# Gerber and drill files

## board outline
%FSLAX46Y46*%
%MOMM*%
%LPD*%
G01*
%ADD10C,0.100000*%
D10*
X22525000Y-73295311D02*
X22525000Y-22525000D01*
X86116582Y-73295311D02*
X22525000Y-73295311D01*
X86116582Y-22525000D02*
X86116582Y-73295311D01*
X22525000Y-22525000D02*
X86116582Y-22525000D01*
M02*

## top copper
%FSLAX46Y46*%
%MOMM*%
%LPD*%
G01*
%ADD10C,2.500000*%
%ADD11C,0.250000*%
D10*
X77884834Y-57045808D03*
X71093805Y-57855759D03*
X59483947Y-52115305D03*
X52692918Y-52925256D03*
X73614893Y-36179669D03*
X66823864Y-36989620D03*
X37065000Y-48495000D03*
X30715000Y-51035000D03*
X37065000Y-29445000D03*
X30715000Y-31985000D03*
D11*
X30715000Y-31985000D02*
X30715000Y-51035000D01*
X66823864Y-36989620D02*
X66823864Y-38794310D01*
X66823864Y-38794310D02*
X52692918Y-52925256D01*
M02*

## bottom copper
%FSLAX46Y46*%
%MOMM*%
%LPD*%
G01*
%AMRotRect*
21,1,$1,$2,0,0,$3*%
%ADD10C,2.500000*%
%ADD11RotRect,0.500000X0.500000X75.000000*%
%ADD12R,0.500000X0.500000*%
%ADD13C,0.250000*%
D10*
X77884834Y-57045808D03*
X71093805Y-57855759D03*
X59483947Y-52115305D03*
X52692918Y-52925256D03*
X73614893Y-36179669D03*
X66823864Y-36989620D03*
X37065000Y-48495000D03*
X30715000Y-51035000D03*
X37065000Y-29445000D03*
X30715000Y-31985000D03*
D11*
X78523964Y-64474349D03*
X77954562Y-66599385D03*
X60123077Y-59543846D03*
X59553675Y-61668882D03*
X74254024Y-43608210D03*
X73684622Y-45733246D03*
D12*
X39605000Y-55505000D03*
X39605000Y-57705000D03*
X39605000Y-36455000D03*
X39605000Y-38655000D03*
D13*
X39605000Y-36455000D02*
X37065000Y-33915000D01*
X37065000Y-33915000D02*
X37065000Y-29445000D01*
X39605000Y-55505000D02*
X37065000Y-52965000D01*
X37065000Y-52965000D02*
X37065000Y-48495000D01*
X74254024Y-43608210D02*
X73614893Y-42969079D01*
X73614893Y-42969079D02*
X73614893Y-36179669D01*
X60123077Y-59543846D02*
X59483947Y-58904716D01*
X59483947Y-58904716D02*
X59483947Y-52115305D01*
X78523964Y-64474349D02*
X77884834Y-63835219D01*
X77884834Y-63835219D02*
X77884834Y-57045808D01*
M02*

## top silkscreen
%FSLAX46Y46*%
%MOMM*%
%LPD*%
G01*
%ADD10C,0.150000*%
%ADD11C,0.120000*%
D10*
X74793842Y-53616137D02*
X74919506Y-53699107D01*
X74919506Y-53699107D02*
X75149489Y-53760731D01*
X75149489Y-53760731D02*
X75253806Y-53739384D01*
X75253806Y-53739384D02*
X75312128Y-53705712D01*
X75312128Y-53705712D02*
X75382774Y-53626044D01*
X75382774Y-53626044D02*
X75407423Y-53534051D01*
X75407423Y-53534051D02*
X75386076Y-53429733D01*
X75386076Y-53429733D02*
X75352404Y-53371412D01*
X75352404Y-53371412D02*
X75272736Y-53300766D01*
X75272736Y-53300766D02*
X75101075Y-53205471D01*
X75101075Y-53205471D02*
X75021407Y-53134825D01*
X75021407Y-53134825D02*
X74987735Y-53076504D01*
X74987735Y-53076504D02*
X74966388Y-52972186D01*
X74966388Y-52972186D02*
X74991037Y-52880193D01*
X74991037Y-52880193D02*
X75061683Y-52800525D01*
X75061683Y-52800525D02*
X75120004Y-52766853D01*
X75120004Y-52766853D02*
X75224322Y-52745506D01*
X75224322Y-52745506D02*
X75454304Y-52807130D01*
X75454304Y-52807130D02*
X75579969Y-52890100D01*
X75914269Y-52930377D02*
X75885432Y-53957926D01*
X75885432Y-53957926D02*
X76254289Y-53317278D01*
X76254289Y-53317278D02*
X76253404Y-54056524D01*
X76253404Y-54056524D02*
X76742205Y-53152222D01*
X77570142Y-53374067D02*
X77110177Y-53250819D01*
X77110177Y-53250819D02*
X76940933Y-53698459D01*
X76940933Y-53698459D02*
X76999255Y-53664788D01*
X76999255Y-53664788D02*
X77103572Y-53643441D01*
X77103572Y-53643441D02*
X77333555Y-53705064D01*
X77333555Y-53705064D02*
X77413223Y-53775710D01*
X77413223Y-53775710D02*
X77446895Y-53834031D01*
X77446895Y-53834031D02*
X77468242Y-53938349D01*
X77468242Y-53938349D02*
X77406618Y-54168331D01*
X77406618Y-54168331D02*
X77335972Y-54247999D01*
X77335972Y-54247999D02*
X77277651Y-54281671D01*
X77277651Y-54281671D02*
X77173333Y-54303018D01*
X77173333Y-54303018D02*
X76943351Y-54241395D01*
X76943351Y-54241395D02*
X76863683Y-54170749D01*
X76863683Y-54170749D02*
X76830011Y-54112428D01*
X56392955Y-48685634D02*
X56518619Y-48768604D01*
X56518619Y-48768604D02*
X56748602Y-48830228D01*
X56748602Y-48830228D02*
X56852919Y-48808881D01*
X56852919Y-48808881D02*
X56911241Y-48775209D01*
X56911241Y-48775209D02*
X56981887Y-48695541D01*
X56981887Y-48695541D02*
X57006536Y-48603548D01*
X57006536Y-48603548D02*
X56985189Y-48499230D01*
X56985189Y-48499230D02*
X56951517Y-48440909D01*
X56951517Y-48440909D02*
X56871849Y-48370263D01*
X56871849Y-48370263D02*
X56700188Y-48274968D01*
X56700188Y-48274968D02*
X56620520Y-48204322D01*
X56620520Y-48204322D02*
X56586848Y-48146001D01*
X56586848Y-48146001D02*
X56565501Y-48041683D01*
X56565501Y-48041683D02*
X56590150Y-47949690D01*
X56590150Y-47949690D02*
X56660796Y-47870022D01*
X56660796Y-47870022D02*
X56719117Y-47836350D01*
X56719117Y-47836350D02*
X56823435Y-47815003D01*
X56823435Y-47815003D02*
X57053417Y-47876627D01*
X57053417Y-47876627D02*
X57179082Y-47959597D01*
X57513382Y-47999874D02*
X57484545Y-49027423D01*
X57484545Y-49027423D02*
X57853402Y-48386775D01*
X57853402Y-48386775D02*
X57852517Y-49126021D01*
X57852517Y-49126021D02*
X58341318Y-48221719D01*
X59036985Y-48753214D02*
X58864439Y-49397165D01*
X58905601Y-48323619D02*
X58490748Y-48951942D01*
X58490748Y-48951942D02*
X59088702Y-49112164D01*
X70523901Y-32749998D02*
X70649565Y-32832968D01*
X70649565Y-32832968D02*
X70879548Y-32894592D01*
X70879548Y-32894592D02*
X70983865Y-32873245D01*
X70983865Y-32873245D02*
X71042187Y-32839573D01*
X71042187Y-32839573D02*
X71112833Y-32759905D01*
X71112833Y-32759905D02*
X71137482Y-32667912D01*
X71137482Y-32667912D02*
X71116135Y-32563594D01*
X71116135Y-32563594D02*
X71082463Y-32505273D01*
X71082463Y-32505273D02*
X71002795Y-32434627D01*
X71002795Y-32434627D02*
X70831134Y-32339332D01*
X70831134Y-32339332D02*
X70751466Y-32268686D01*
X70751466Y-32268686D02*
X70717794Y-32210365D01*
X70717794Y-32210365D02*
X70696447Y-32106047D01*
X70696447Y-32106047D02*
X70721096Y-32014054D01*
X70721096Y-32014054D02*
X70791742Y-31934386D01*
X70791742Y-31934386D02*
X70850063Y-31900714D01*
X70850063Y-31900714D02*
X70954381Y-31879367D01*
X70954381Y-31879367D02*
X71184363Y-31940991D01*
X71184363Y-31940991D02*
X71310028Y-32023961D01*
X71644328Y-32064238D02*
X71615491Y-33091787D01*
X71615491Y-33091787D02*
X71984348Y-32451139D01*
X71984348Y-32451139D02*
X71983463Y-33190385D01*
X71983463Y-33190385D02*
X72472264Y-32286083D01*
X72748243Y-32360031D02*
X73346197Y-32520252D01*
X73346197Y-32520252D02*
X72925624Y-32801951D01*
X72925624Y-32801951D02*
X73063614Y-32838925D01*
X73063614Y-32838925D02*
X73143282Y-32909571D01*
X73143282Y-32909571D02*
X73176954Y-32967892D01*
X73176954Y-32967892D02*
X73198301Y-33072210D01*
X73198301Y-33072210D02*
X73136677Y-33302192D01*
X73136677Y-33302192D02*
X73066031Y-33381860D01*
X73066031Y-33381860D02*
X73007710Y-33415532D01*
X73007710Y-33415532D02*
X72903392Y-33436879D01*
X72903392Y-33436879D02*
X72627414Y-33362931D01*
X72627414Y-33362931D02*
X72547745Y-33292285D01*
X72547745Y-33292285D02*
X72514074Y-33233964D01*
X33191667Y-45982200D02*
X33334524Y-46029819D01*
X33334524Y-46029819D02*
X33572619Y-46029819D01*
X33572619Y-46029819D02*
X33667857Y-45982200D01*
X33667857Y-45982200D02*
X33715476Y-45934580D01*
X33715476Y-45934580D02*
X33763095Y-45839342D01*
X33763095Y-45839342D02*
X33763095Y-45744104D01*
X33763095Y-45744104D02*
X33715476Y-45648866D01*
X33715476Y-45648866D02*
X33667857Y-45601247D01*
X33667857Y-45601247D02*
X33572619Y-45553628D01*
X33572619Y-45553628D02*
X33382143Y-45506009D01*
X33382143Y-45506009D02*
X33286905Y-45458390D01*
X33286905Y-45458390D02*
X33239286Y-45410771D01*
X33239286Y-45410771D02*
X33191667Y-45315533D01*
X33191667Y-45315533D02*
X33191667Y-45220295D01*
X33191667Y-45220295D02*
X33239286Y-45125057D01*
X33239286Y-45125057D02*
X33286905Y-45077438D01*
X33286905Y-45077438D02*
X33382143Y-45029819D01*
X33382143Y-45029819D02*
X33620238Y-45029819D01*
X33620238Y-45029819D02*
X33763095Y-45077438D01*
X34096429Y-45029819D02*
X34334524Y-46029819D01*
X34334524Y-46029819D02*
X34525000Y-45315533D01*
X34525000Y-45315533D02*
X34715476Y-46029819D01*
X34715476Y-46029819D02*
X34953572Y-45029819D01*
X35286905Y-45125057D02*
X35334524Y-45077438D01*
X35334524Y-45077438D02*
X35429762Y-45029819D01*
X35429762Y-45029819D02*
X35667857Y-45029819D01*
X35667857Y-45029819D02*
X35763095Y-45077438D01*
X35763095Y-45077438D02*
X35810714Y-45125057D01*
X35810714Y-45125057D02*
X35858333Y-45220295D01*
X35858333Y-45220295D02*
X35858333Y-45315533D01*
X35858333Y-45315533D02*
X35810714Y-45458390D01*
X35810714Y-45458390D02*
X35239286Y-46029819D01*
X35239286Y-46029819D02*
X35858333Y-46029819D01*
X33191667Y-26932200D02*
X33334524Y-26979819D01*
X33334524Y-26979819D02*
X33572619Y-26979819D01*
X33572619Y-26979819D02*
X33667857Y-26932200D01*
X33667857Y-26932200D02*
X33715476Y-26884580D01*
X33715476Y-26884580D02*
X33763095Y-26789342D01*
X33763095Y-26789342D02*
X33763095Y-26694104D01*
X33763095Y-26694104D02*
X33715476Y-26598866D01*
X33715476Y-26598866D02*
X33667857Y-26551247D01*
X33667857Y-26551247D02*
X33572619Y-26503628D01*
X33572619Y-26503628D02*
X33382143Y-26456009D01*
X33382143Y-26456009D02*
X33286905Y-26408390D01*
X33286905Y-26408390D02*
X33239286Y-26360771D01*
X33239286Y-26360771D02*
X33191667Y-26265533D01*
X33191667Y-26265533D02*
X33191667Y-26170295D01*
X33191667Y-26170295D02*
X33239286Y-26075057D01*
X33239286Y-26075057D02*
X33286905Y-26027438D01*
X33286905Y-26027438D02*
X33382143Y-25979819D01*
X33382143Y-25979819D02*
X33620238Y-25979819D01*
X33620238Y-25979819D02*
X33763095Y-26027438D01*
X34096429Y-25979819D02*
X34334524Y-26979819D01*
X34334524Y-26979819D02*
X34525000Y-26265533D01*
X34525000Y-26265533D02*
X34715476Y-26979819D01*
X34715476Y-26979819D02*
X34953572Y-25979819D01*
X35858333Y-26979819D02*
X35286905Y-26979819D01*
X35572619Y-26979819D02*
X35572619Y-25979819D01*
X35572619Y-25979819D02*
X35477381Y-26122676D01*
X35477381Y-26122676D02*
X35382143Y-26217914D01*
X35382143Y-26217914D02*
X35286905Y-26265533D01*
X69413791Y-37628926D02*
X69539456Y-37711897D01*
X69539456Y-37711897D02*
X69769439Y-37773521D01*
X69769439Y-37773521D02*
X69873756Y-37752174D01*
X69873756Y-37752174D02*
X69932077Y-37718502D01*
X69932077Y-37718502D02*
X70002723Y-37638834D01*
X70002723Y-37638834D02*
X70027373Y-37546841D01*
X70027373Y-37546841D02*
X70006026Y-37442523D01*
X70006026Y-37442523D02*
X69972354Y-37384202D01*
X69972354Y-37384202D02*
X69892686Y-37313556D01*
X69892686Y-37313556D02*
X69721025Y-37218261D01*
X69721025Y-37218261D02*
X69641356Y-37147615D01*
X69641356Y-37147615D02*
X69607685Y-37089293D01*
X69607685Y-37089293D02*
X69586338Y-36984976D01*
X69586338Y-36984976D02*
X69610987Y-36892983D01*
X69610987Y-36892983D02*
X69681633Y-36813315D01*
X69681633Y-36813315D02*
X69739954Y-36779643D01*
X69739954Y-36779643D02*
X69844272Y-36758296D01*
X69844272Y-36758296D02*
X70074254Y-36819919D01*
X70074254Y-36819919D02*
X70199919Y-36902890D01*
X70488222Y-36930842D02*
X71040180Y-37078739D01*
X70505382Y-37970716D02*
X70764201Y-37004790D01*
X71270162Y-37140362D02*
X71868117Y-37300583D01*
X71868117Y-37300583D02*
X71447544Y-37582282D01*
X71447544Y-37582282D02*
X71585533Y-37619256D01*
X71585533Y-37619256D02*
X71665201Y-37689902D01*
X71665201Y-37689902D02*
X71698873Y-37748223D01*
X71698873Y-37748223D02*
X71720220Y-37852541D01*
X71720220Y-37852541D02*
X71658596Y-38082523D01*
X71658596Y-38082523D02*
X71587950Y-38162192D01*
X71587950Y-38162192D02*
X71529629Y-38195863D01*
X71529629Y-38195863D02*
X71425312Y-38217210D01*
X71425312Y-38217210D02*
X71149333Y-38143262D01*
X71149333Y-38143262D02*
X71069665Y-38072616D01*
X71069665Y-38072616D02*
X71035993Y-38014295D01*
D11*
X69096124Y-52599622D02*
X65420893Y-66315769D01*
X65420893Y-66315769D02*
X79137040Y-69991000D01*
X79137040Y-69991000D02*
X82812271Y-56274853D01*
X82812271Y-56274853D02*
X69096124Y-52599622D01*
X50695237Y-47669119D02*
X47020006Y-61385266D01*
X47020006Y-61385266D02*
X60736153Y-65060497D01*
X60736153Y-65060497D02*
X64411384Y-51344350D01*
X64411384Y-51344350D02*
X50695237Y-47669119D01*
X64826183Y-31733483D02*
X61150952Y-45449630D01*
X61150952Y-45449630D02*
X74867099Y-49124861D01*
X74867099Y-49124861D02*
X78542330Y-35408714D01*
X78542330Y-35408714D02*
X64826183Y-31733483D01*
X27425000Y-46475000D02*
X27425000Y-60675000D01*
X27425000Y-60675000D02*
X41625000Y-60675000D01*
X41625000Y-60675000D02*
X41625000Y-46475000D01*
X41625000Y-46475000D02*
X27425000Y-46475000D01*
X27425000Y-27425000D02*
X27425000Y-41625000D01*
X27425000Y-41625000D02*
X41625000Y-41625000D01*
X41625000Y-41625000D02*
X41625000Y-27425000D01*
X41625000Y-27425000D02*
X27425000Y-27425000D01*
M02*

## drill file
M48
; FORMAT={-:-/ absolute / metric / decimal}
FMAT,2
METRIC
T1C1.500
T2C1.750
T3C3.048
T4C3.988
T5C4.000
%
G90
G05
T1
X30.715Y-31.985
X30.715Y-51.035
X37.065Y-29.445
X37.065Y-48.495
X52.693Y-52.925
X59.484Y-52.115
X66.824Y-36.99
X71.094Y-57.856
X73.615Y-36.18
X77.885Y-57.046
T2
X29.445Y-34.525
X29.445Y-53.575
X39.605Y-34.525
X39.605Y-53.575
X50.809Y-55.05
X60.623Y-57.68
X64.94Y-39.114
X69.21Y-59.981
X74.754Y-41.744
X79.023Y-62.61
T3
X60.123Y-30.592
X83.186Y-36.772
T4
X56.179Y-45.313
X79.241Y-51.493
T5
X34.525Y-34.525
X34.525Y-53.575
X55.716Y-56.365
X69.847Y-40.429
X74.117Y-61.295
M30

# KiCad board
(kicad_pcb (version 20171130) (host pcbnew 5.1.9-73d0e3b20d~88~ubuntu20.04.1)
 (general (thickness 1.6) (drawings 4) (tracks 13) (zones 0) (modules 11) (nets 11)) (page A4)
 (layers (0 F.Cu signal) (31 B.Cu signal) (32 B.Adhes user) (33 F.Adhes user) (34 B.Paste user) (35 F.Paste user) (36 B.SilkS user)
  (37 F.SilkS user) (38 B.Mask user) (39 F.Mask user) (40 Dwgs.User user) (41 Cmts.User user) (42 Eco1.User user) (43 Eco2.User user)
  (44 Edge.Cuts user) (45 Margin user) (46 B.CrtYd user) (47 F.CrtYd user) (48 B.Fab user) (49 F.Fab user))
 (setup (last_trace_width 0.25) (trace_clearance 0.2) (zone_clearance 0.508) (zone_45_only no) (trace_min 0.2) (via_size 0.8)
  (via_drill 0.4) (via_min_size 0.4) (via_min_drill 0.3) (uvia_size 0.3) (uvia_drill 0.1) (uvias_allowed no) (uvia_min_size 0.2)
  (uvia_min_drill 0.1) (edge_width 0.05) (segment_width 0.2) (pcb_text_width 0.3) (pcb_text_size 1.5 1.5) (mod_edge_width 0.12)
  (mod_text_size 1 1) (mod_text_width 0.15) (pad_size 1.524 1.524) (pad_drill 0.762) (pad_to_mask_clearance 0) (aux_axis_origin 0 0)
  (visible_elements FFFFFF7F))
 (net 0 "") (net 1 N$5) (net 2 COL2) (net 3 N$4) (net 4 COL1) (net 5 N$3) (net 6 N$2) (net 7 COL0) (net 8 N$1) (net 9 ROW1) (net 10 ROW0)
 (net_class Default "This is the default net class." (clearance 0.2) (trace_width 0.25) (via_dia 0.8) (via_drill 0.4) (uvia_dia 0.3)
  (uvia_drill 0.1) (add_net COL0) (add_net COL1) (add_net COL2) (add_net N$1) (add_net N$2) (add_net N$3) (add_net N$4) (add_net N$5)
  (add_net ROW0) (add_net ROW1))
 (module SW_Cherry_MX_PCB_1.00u (layer F.Cu) (at 74.116582 61.295311 345)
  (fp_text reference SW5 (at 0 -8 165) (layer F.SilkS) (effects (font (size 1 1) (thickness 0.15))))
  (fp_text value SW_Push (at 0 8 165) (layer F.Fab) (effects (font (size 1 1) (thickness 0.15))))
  (fp_line (start -7.1 -7.1) (end -7.1 7.1) (layer F.SilkS) (width 0.12))
  (fp_line (start -7.1 7.1) (end 7.1 7.1) (layer F.SilkS) (width 0.12))
  (fp_line (start 7.1 7.1) (end 7.1 -7.1) (layer F.SilkS) (width 0.12))
  (fp_line (start 7.1 -7.1) (end -7.1 -7.1) (layer F.SilkS) (width 0.12))
  (pad "" np_thru_hole circle (at 5.08 0 345) (size 1.75 1.75) (drill 1.75) (layers *.Cu *.Mask))
  (pad "" np_thru_hole circle (at -5.08 0 345) (size 1.75 1.75) (drill 1.75) (layers *.Cu *.Mask))
  (pad "" np_thru_hole circle (at 0 0 345) (size 4 4) (drill 4) (layers *.Cu *.Mask))
  (pad 2 thru_hole circle (at 2.54 -5.08 345) (size 2.5 2.5) (drill 1.5) (layers *.Cu B.Mask) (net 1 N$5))
  (pad 1 thru_hole circle (at -3.81 -2.54 345) (size 2.5 2.5) (drill 1.5) (layers *.Cu B.Mask) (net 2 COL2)))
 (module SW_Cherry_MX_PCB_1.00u (layer F.Cu) (at 55.715695 56.364808 345)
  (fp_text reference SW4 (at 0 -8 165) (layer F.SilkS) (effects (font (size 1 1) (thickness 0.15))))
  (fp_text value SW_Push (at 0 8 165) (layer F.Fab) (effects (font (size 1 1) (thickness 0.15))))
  (fp_line (start -7.1 -7.1) (end -7.1 7.1) (layer F.SilkS) (width 0.12))
  (fp_line (start -7.1 7.1) (end 7.1 7.1) (layer F.SilkS) (width 0.12))
  (fp_line (start 7.1 7.1) (end 7.1 -7.1) (layer F.SilkS) (width 0.12))
  (fp_line (start 7.1 -7.1) (end -7.1 -7.1) (layer F.SilkS) (width 0.12))
  (pad "" np_thru_hole circle (at 5.08 0 345) (size 1.75 1.75) (drill 1.75) (layers *.Cu *.Mask))
  (pad "" np_thru_hole circle (at -5.08 0 345) (size 1.75 1.75) (drill 1.75) (layers *.Cu *.Mask))
  (pad "" np_thru_hole circle (at 0 0 345) (size 4 4) (drill 4) (layers *.Cu *.Mask))
  (pad 2 thru_hole circle (at 2.54 -5.08 345) (size 2.5 2.5) (drill 1.5) (layers *.Cu B.Mask) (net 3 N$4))
  (pad 1 thru_hole circle (at -3.81 -2.54 345) (size 2.5 2.5) (drill 1.5) (layers *.Cu B.Mask) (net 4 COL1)))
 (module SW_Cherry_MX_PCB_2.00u (layer F.Cu) (at 69.846641 40.429172 345)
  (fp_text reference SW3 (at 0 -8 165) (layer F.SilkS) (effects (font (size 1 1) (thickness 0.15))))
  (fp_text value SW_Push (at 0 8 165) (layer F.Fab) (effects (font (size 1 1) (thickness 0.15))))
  (fp_line (start -7.1 -7.1) (end -7.1 7.1) (layer F.SilkS) (width 0.12))
  (fp_line (start -7.1 7.1) (end 7.1 7.1) (layer F.SilkS) (width 0.12))
  (fp_line (start 7.1 7.1) (end 7.1 -7.1) (layer F.SilkS) (width 0.12))
  (fp_line (start 7.1 -7.1) (end -7.1 -7.1) (layer F.SilkS) (width 0.12))
  (pad "" np_thru_hole circle (at 5.08 0 345) (size 1.75 1.75) (drill 1.75) (layers *.Cu *.Mask))
  (pad "" np_thru_hole circle (at -5.08 0 345) (size 1.75 1.75) (drill 1.75) (layers *.Cu *.Mask))
  (pad "" np_thru_hole circle (at 0 0 345) (size 4 4) (drill 4) (layers *.Cu *.Mask))
  (pad 2 thru_hole circle (at 2.54 -5.08 345) (size 2.5 2.5) (drill 1.5) (layers *.Cu B.Mask) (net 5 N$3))
  (pad 1 thru_hole circle (at -3.81 -2.54 345) (size 2.5 2.5) (drill 1.5) (layers *.Cu B.Mask) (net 4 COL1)))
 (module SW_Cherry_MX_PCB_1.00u (layer F.Cu) (at 34.525 53.575)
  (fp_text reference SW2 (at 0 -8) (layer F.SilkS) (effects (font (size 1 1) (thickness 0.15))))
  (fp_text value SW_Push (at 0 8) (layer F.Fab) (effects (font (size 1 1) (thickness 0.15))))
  (fp_line (start -7.1 -7.1) (end -7.1 7.1) (layer F.SilkS) (width 0.12))
  (fp_line (start -7.1 7.1) (end 7.1 7.1) (layer F.SilkS) (width 0.12))
  (fp_line (start 7.1 7.1) (end 7.1 -7.1) (layer F.SilkS) (width 0.12))
  (fp_line (start 7.1 -7.1) (end -7.1 -7.1) (layer F.SilkS) (width 0.12))
  (pad "" np_thru_hole circle (at 5.08 0) (size 1.75 1.75) (drill 1.75) (layers *.Cu *.Mask))
  (pad "" np_thru_hole circle (at -5.08 0) (size 1.75 1.75) (drill 1.75) (layers *.Cu *.Mask))
  (pad "" np_thru_hole circle (at 0 0) (size 4 4) (drill 4) (layers *.Cu *.Mask))
  (pad 2 thru_hole circle (at 2.54 -5.08) (size 2.5 2.5) (drill 1.5) (layers *.Cu B.Mask) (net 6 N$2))
  (pad 1 thru_hole circle (at -3.81 -2.54) (size 2.5 2.5) (drill 1.5) (layers *.Cu B.Mask) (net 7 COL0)))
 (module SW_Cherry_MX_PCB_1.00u (layer F.Cu) (at 34.525 34.525)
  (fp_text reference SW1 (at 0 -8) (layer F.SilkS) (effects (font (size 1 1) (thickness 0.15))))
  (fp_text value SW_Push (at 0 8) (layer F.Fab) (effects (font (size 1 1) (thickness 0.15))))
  (fp_line (start -7.1 -7.1) (end -7.1 7.1) (layer F.SilkS) (width 0.12))
  (fp_line (start -7.1 7.1) (end 7.1 7.1) (layer F.SilkS) (width 0.12))
  (fp_line (start 7.1 7.1) (end 7.1 -7.1) (layer F.SilkS) (width 0.12))
  (fp_line (start 7.1 -7.1) (end -7.1 -7.1) (layer F.SilkS) (width 0.12))
  (pad "" np_thru_hole circle (at 5.08 0) (size 1.75 1.75) (drill 1.75) (layers *.Cu *.Mask))
  (pad "" np_thru_hole circle (at -5.08 0) (size 1.75 1.75) (drill 1.75) (layers *.Cu *.Mask))
  (pad "" np_thru_hole circle (at 0 0) (size 4 4) (drill 4) (layers *.Cu *.Mask))
  (pad 2 thru_hole circle (at 2.54 -5.08) (size 2.5 2.5) (drill 1.5) (layers *.Cu B.Mask) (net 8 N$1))
  (pad 1 thru_hole circle (at -3.81 -2.54) (size 2.5 2.5) (drill 1.5) (layers *.Cu B.Mask) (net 7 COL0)))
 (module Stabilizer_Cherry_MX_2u (layer F.Cu) (at 69.846641 40.429172 345)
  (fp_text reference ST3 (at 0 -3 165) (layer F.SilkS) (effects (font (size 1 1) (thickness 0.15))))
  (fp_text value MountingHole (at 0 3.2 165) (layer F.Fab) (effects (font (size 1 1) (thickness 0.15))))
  (pad ~ np_thru_hole circle (at 11.938 -6.985 345) (size 3.048 3.048) (drill 3.048) (layers *.Cu *.Mask))
  (pad ~ np_thru_hole circle (at -11.938 -6.985 345) (size 3.048 3.048) (drill 3.048) (layers *.Cu *.Mask))
  (pad ~ np_thru_hole circle (at 11.938 8.255 345) (size 3.9878 3.9878) (drill 3.9878) (layers *.Cu *.Mask))
  (pad ~ np_thru_hole circle (at -11.938 8.255 345) (size 3.9878 3.9878) (drill 3.9878) (layers *.Cu *.Mask)))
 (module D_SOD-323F (layer B.Cu) (at 78.239263 65.536867 75)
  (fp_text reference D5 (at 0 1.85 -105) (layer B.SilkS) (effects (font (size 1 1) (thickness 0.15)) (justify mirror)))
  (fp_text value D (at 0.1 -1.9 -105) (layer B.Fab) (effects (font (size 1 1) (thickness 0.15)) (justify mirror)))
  (pad 2 smd rect (at 1.1 0 75) (size 0.5 0.5) (layers B.Cu B.Paste B.Mask) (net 1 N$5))
  (pad 1 smd rect (at -1.1 0 75) (size 0.5 0.5) (layers B.Cu B.Paste B.Mask) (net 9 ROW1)))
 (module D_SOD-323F (layer B.Cu) (at 59.838376 60.606364 75)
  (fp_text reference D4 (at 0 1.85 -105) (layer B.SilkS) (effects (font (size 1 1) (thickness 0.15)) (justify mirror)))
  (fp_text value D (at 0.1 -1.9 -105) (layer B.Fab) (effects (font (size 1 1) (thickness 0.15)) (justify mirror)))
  (pad 2 smd rect (at 1.1 0 75) (size 0.5 0.5) (layers B.Cu B.Paste B.Mask) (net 3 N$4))
  (pad 1 smd rect (at -1.1 0 75) (size 0.5 0.5) (layers B.Cu B.Paste B.Mask) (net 9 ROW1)))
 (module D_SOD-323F (layer B.Cu) (at 73.969323 44.670728 75)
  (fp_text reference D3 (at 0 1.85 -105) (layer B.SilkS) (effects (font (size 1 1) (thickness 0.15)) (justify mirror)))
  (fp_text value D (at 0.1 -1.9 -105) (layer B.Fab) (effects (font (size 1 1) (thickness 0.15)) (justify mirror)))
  (pad 2 smd rect (at 1.1 0 75) (size 0.5 0.5) (layers B.Cu B.Paste B.Mask) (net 5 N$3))
  (pad 1 smd rect (at -1.1 0 75) (size 0.5 0.5) (layers B.Cu B.Paste B.Mask) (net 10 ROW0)))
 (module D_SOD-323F (layer B.Cu) (at 39.605 56.605 90)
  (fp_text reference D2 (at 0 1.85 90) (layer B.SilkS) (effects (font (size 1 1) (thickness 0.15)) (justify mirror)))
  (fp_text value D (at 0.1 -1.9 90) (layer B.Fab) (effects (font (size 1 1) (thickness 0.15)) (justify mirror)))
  (pad 2 smd rect (at 1.1 0 90) (size 0.5 0.5) (layers B.Cu B.Paste B.Mask) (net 6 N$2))
  (pad 1 smd rect (at -1.1 0 90) (size 0.5 0.5) (layers B.Cu B.Paste B.Mask) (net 9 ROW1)))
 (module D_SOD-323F (layer B.Cu) (at 39.605 37.555 90)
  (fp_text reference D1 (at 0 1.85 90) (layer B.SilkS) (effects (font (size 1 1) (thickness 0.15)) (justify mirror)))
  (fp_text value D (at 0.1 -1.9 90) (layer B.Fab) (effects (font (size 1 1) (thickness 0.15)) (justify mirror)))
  (pad 2 smd rect (at 1.1 0 90) (size 0.5 0.5) (layers B.Cu B.Paste B.Mask) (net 8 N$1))
  (pad 1 smd rect (at -1.1 0 90) (size 0.5 0.5) (layers B.Cu B.Paste B.Mask) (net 10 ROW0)))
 (gr_line (start 22.525 73.295311) (end 22.525 22.525) (layer Edge.Cuts) (width 0.1))
 (gr_line (start 86.116582 73.295311) (end 22.525 73.295311) (layer Edge.Cuts) (width 0.1))
 (gr_line (start 86.116582 22.525) (end 86.116582 73.295311) (layer Edge.Cuts) (width 0.1))
 (gr_line (start 22.525 22.525) (end 86.116582 22.525) (layer Edge.Cuts) (width 0.1))
 (segment (start 30.715 31.985) (end 30.715 51.035) (width 0.25) (layer F.Cu) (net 7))
 (segment (start 66.823864 36.98962) (end 66.823864 38.79431) (width 0.25) (layer F.Cu) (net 4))
 (segment (start 66.823864 38.79431) (end 52.692918 52.925256) (width 0.25) (layer F.Cu) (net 4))
 (segment (start 39.605 36.455) (end 37.065 33.915) (width 0.25) (layer B.Cu) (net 8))
 (segment (start 37.065 33.915) (end 37.065 29.445) (width 0.25) (layer B.Cu) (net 8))
 (segment (start 39.605 55.505) (end 37.065 52.965) (width 0.25) (layer B.Cu) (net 6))
 (segment (start 37.065 52.965) (end 37.065 48.495) (width 0.25) (layer B.Cu) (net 6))
 (segment (start 74.254024 43.60821) (end 73.614893 42.969079) (width 0.25) (layer B.Cu) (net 5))
 (segment (start 73.614893 42.969079) (end 73.614893 36.179669) (width 0.25) (layer B.Cu) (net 5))
 (segment (start 60.123077 59.543846) (end 59.483947 58.904716) (width 0.25) (layer B.Cu) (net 3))
 (segment (start 59.483947 58.904716) (end 59.483947 52.115305) (width 0.25) (layer B.Cu) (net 3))
 (segment (start 78.523964 64.474349) (end 77.884834 63.835219) (width 0.25) (layer B.Cu) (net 1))
 (segment (start 77.884834 63.835219) (end 77.884834 57.045808) (width 0.25) (layer B.Cu) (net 1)))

